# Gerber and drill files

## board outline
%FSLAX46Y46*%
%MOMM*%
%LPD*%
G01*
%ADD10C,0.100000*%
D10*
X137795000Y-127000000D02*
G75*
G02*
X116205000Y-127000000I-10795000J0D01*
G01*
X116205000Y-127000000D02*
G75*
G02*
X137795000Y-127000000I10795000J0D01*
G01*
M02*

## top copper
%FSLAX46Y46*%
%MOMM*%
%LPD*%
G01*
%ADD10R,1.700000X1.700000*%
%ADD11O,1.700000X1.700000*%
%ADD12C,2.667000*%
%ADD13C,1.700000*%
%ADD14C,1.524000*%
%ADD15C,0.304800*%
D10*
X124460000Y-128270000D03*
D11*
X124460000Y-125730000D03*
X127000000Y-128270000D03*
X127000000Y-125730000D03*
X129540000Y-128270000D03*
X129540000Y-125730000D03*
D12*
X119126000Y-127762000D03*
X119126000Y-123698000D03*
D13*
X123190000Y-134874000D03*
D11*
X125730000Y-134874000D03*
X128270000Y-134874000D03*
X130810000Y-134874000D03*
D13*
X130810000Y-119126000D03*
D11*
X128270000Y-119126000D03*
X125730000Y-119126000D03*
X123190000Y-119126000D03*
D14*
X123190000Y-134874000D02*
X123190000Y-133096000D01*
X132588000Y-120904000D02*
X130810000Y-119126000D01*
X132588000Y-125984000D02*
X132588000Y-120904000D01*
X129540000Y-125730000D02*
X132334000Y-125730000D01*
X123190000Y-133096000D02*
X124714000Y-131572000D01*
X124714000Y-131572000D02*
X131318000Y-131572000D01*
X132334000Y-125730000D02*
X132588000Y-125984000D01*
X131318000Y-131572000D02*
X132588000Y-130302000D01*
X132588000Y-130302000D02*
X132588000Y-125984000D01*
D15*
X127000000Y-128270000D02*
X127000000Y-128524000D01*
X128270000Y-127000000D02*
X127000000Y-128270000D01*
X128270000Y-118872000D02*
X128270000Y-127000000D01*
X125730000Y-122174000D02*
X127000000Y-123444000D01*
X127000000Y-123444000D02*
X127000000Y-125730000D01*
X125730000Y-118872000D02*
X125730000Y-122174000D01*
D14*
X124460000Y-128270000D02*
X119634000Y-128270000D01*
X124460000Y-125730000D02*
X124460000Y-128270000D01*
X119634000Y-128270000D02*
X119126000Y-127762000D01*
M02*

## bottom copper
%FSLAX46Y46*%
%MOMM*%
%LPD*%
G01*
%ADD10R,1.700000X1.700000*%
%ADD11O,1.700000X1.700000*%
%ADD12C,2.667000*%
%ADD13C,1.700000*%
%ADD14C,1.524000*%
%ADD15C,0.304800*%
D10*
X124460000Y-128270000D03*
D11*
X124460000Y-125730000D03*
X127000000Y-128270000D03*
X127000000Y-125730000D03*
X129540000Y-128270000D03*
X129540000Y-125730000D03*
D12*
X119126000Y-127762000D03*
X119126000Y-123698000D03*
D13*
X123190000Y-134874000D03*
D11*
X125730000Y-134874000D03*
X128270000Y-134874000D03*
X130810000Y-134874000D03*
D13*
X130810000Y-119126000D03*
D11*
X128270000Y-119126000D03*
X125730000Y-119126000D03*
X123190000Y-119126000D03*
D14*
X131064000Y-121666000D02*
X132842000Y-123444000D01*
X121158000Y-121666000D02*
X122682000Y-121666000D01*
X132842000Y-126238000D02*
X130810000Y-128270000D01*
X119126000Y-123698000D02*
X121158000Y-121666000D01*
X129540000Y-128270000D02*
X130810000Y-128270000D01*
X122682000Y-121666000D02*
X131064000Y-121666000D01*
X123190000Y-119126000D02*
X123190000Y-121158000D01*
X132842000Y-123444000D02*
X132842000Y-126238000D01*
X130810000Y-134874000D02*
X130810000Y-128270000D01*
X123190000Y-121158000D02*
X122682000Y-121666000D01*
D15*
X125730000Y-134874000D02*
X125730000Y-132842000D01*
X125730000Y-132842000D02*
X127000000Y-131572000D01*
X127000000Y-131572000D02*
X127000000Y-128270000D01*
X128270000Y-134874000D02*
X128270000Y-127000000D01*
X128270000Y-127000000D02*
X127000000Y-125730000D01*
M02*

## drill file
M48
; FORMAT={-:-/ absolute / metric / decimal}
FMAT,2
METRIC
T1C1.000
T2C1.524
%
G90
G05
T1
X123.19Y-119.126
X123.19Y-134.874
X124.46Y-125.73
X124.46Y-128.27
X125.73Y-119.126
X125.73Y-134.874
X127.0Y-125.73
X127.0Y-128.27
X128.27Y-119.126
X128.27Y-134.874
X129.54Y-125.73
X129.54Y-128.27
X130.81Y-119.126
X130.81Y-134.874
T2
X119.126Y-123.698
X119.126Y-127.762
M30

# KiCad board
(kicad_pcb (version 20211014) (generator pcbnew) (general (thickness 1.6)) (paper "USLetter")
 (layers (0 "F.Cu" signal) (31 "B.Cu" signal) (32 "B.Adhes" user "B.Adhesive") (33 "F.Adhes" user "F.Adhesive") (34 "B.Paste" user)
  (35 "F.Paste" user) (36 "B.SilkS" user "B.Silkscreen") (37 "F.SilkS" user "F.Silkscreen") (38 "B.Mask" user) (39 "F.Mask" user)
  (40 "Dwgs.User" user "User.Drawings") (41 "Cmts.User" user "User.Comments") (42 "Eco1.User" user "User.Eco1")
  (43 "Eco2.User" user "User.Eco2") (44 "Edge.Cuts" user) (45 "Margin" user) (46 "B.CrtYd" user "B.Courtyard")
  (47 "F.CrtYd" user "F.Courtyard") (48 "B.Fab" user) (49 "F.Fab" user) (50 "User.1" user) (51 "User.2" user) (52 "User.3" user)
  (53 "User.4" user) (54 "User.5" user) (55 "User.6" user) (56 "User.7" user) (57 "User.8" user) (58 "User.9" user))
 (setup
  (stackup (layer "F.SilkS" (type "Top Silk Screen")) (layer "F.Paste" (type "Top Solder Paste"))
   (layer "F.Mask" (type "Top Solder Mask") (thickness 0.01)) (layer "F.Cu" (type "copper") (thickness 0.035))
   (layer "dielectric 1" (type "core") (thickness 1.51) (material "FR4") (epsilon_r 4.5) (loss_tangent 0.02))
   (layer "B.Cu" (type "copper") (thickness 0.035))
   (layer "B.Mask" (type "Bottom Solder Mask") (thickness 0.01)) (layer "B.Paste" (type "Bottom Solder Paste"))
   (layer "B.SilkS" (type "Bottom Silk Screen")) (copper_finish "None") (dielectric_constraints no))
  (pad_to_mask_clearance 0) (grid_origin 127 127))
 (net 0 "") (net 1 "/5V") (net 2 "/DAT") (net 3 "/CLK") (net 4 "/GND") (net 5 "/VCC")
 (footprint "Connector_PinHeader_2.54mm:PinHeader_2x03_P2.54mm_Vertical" (layer "F.Cu") (at 124.46 128.27 90)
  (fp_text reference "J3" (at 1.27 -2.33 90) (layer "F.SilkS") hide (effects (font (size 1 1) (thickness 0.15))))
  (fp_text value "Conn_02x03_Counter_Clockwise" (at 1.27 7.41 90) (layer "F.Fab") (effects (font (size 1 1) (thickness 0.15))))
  (pad "1" thru_hole rect (at 0 0 90) (size 1.7 1.7) (drill 1) (layers *.Cu *.Mask) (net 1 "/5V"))
  (pad "2" thru_hole oval (at 2.54 0 90) (size 1.7 1.7) (drill 1) (layers *.Cu *.Mask) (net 1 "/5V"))
  (pad "3" thru_hole oval (at 0 2.54 90) (size 1.7 1.7) (drill 1) (layers *.Cu *.Mask) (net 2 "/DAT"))
  (pad "4" thru_hole oval (at 2.54 2.54 90) (size 1.7 1.7) (drill 1) (layers *.Cu *.Mask) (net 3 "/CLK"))
  (pad "5" thru_hole oval (at 0 5.08 90) (size 1.7 1.7) (drill 1) (layers *.Cu *.Mask) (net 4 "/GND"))
  (pad "6" thru_hole oval (at 2.54 5.08 90) (size 1.7 1.7) (drill 1) (layers *.Cu *.Mask) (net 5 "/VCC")))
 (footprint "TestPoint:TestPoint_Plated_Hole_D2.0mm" (layer "F.Cu") (at 119.126 127.762)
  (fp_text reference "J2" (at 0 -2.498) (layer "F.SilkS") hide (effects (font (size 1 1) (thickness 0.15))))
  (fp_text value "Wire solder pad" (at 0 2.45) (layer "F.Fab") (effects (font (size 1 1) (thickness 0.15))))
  (pad "1" thru_hole circle (at 0 0) (size 2.667 2.667) (drill 1.524) (layers *.Cu *.Mask) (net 1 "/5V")))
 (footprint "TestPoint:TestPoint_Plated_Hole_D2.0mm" (layer "F.Cu") (at 119.126 123.698)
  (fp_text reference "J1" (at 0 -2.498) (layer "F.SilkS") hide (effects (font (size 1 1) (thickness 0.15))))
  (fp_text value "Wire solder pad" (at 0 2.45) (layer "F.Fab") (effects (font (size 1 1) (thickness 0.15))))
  (pad "1" thru_hole circle (at 0 0) (size 2.667 2.667) (drill 1.524) (layers *.Cu *.Mask) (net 4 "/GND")))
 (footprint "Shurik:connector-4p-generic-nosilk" (layer "F.Cu") (at 123.19 134.874 90)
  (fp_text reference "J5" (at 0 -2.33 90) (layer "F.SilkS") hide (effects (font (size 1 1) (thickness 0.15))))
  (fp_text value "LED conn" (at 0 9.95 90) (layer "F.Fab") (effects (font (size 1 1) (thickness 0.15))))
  (pad "1" thru_hole circle (at 0 0 90) (size 1.7 1.7) (drill 1) (layers *.Cu *.Mask) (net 5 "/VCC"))
  (pad "2" thru_hole oval (at 0 2.54 90) (size 1.7 1.7) (drill 1) (layers *.Cu *.Mask) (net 2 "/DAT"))
  (pad "3" thru_hole oval (at 0 5.08 90) (size 1.7 1.7) (drill 1) (layers *.Cu *.Mask) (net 3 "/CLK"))
  (pad "4" thru_hole oval (at 0 7.62 90) (size 1.7 1.7) (drill 1) (layers *.Cu *.Mask) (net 4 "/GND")))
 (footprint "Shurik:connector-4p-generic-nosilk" (layer "F.Cu") (at 130.81 119.126 -90)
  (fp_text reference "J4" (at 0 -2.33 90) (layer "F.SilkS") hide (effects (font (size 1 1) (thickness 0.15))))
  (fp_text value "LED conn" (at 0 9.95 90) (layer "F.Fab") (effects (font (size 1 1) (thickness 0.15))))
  (pad "1" thru_hole circle (at 0 0 270) (size 1.7 1.7) (drill 1) (layers *.Cu *.Mask) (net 5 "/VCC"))
  (pad "2" thru_hole oval (at 0 2.54 270) (size 1.7 1.7) (drill 1) (layers *.Cu *.Mask) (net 2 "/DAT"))
  (pad "3" thru_hole oval (at 0 5.08 270) (size 1.7 1.7) (drill 1) (layers *.Cu *.Mask) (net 3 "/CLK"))
  (pad "4" thru_hole oval (at 0 7.62 270) (size 1.7 1.7) (drill 1) (layers *.Cu *.Mask) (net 4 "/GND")))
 (gr_arc (start 137.795 127) (mid 127 137.795) (end 116.205 127) (layer "Edge.Cuts") (width 0.1))
 (gr_arc (start 116.205 127) (mid 127 116.205) (end 137.795 127) (layer "Edge.Cuts") (width 0.1))
 (segment (start 131.064 121.666) (end 132.842 123.444) (width 1.524) (layer "B.Cu") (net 4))
 (segment (start 121.158 121.666) (end 122.682 121.666) (width 1.524) (layer "B.Cu") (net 4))
 (segment (start 132.842 126.238) (end 130.81 128.27) (width 1.524) (layer "B.Cu") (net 4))
 (segment (start 119.126 123.698) (end 121.158 121.666) (width 1.524) (layer "B.Cu") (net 4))
 (segment (start 129.54 128.27) (end 130.81 128.27) (width 1.524) (layer "B.Cu") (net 4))
 (segment (start 122.682 121.666) (end 131.064 121.666) (width 1.524) (layer "B.Cu") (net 4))
 (segment (start 123.19 119.126) (end 123.19 121.158) (width 1.524) (layer "B.Cu") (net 4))
 (segment (start 132.842 123.444) (end 132.842 126.238) (width 1.524) (layer "B.Cu") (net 4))
 (segment (start 130.81 134.874) (end 130.81 128.27) (width 1.524) (layer "B.Cu") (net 4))
 (segment (start 123.19 121.158) (end 122.682 121.666) (width 1.524) (layer "B.Cu") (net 4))
 (segment (start 123.19 134.874) (end 123.19 133.096) (width 1.524) (layer "F.Cu") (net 5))
 (segment (start 132.588 120.904) (end 130.81 119.126) (width 1.524) (layer "F.Cu") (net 5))
 (segment (start 132.588 125.984) (end 132.588 120.904) (width 1.524) (layer "F.Cu") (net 5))
 (segment (start 129.54 125.73) (end 132.334 125.73) (width 1.524) (layer "F.Cu") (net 5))
 (segment (start 123.19 133.096) (end 124.714 131.572) (width 1.524) (layer "F.Cu") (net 5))
 (segment (start 124.714 131.572) (end 131.318 131.572) (width 1.524) (layer "F.Cu") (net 5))
 (segment (start 132.334 125.73) (end 132.588 125.984) (width 1.524) (layer "F.Cu") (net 5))
 (segment (start 131.318 131.572) (end 132.588 130.302) (width 1.524) (layer "F.Cu") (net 5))
 (segment (start 132.588 130.302) (end 132.588 125.984) (width 1.524) (layer "F.Cu") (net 5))
 (segment (start 127 128.27) (end 127 128.524) (width 0.3048) (layer "F.Cu") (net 2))
 (segment (start 128.27 127) (end 127 128.27) (width 0.3048) (layer "F.Cu") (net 2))
 (segment (start 128.27 118.872) (end 128.27 127) (width 0.3048) (layer "F.Cu") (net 2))
 (segment (start 125.73 134.874) (end 125.73 132.842) (width 0.3048) (layer "B.Cu") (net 2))
 (segment (start 125.73 132.842) (end 127 131.572) (width 0.3048) (layer "B.Cu") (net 2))
 (segment (start 127 131.572) (end 127 128.27) (width 0.3048) (layer "B.Cu") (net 2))
 (segment (start 125.73 122.174) (end 127 123.444) (width 0.3048) (layer "F.Cu") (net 3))
 (segment (start 127 123.444) (end 127 125.73) (width 0.3048) (layer "F.Cu") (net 3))
 (segment (start 125.73 118.872) (end 125.73 122.174) (width 0.3048) (layer "F.Cu") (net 3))
 (segment (start 128.27 134.874) (end 128.27 127) (width 0.3048) (layer "B.Cu") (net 3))
 (segment (start 128.27 127) (end 127 125.73) (width 0.3048) (layer "B.Cu") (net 3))
 (segment (start 124.46 128.27) (end 119.634 128.27) (width 1.524) (layer "F.Cu") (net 1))
 (segment (start 124.46 125.73) (end 124.46 128.27) (width 1.524) (layer "F.Cu") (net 1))
 (segment (start 119.634 128.27) (end 119.126 127.762) (width 1.524) (layer "F.Cu") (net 1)))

